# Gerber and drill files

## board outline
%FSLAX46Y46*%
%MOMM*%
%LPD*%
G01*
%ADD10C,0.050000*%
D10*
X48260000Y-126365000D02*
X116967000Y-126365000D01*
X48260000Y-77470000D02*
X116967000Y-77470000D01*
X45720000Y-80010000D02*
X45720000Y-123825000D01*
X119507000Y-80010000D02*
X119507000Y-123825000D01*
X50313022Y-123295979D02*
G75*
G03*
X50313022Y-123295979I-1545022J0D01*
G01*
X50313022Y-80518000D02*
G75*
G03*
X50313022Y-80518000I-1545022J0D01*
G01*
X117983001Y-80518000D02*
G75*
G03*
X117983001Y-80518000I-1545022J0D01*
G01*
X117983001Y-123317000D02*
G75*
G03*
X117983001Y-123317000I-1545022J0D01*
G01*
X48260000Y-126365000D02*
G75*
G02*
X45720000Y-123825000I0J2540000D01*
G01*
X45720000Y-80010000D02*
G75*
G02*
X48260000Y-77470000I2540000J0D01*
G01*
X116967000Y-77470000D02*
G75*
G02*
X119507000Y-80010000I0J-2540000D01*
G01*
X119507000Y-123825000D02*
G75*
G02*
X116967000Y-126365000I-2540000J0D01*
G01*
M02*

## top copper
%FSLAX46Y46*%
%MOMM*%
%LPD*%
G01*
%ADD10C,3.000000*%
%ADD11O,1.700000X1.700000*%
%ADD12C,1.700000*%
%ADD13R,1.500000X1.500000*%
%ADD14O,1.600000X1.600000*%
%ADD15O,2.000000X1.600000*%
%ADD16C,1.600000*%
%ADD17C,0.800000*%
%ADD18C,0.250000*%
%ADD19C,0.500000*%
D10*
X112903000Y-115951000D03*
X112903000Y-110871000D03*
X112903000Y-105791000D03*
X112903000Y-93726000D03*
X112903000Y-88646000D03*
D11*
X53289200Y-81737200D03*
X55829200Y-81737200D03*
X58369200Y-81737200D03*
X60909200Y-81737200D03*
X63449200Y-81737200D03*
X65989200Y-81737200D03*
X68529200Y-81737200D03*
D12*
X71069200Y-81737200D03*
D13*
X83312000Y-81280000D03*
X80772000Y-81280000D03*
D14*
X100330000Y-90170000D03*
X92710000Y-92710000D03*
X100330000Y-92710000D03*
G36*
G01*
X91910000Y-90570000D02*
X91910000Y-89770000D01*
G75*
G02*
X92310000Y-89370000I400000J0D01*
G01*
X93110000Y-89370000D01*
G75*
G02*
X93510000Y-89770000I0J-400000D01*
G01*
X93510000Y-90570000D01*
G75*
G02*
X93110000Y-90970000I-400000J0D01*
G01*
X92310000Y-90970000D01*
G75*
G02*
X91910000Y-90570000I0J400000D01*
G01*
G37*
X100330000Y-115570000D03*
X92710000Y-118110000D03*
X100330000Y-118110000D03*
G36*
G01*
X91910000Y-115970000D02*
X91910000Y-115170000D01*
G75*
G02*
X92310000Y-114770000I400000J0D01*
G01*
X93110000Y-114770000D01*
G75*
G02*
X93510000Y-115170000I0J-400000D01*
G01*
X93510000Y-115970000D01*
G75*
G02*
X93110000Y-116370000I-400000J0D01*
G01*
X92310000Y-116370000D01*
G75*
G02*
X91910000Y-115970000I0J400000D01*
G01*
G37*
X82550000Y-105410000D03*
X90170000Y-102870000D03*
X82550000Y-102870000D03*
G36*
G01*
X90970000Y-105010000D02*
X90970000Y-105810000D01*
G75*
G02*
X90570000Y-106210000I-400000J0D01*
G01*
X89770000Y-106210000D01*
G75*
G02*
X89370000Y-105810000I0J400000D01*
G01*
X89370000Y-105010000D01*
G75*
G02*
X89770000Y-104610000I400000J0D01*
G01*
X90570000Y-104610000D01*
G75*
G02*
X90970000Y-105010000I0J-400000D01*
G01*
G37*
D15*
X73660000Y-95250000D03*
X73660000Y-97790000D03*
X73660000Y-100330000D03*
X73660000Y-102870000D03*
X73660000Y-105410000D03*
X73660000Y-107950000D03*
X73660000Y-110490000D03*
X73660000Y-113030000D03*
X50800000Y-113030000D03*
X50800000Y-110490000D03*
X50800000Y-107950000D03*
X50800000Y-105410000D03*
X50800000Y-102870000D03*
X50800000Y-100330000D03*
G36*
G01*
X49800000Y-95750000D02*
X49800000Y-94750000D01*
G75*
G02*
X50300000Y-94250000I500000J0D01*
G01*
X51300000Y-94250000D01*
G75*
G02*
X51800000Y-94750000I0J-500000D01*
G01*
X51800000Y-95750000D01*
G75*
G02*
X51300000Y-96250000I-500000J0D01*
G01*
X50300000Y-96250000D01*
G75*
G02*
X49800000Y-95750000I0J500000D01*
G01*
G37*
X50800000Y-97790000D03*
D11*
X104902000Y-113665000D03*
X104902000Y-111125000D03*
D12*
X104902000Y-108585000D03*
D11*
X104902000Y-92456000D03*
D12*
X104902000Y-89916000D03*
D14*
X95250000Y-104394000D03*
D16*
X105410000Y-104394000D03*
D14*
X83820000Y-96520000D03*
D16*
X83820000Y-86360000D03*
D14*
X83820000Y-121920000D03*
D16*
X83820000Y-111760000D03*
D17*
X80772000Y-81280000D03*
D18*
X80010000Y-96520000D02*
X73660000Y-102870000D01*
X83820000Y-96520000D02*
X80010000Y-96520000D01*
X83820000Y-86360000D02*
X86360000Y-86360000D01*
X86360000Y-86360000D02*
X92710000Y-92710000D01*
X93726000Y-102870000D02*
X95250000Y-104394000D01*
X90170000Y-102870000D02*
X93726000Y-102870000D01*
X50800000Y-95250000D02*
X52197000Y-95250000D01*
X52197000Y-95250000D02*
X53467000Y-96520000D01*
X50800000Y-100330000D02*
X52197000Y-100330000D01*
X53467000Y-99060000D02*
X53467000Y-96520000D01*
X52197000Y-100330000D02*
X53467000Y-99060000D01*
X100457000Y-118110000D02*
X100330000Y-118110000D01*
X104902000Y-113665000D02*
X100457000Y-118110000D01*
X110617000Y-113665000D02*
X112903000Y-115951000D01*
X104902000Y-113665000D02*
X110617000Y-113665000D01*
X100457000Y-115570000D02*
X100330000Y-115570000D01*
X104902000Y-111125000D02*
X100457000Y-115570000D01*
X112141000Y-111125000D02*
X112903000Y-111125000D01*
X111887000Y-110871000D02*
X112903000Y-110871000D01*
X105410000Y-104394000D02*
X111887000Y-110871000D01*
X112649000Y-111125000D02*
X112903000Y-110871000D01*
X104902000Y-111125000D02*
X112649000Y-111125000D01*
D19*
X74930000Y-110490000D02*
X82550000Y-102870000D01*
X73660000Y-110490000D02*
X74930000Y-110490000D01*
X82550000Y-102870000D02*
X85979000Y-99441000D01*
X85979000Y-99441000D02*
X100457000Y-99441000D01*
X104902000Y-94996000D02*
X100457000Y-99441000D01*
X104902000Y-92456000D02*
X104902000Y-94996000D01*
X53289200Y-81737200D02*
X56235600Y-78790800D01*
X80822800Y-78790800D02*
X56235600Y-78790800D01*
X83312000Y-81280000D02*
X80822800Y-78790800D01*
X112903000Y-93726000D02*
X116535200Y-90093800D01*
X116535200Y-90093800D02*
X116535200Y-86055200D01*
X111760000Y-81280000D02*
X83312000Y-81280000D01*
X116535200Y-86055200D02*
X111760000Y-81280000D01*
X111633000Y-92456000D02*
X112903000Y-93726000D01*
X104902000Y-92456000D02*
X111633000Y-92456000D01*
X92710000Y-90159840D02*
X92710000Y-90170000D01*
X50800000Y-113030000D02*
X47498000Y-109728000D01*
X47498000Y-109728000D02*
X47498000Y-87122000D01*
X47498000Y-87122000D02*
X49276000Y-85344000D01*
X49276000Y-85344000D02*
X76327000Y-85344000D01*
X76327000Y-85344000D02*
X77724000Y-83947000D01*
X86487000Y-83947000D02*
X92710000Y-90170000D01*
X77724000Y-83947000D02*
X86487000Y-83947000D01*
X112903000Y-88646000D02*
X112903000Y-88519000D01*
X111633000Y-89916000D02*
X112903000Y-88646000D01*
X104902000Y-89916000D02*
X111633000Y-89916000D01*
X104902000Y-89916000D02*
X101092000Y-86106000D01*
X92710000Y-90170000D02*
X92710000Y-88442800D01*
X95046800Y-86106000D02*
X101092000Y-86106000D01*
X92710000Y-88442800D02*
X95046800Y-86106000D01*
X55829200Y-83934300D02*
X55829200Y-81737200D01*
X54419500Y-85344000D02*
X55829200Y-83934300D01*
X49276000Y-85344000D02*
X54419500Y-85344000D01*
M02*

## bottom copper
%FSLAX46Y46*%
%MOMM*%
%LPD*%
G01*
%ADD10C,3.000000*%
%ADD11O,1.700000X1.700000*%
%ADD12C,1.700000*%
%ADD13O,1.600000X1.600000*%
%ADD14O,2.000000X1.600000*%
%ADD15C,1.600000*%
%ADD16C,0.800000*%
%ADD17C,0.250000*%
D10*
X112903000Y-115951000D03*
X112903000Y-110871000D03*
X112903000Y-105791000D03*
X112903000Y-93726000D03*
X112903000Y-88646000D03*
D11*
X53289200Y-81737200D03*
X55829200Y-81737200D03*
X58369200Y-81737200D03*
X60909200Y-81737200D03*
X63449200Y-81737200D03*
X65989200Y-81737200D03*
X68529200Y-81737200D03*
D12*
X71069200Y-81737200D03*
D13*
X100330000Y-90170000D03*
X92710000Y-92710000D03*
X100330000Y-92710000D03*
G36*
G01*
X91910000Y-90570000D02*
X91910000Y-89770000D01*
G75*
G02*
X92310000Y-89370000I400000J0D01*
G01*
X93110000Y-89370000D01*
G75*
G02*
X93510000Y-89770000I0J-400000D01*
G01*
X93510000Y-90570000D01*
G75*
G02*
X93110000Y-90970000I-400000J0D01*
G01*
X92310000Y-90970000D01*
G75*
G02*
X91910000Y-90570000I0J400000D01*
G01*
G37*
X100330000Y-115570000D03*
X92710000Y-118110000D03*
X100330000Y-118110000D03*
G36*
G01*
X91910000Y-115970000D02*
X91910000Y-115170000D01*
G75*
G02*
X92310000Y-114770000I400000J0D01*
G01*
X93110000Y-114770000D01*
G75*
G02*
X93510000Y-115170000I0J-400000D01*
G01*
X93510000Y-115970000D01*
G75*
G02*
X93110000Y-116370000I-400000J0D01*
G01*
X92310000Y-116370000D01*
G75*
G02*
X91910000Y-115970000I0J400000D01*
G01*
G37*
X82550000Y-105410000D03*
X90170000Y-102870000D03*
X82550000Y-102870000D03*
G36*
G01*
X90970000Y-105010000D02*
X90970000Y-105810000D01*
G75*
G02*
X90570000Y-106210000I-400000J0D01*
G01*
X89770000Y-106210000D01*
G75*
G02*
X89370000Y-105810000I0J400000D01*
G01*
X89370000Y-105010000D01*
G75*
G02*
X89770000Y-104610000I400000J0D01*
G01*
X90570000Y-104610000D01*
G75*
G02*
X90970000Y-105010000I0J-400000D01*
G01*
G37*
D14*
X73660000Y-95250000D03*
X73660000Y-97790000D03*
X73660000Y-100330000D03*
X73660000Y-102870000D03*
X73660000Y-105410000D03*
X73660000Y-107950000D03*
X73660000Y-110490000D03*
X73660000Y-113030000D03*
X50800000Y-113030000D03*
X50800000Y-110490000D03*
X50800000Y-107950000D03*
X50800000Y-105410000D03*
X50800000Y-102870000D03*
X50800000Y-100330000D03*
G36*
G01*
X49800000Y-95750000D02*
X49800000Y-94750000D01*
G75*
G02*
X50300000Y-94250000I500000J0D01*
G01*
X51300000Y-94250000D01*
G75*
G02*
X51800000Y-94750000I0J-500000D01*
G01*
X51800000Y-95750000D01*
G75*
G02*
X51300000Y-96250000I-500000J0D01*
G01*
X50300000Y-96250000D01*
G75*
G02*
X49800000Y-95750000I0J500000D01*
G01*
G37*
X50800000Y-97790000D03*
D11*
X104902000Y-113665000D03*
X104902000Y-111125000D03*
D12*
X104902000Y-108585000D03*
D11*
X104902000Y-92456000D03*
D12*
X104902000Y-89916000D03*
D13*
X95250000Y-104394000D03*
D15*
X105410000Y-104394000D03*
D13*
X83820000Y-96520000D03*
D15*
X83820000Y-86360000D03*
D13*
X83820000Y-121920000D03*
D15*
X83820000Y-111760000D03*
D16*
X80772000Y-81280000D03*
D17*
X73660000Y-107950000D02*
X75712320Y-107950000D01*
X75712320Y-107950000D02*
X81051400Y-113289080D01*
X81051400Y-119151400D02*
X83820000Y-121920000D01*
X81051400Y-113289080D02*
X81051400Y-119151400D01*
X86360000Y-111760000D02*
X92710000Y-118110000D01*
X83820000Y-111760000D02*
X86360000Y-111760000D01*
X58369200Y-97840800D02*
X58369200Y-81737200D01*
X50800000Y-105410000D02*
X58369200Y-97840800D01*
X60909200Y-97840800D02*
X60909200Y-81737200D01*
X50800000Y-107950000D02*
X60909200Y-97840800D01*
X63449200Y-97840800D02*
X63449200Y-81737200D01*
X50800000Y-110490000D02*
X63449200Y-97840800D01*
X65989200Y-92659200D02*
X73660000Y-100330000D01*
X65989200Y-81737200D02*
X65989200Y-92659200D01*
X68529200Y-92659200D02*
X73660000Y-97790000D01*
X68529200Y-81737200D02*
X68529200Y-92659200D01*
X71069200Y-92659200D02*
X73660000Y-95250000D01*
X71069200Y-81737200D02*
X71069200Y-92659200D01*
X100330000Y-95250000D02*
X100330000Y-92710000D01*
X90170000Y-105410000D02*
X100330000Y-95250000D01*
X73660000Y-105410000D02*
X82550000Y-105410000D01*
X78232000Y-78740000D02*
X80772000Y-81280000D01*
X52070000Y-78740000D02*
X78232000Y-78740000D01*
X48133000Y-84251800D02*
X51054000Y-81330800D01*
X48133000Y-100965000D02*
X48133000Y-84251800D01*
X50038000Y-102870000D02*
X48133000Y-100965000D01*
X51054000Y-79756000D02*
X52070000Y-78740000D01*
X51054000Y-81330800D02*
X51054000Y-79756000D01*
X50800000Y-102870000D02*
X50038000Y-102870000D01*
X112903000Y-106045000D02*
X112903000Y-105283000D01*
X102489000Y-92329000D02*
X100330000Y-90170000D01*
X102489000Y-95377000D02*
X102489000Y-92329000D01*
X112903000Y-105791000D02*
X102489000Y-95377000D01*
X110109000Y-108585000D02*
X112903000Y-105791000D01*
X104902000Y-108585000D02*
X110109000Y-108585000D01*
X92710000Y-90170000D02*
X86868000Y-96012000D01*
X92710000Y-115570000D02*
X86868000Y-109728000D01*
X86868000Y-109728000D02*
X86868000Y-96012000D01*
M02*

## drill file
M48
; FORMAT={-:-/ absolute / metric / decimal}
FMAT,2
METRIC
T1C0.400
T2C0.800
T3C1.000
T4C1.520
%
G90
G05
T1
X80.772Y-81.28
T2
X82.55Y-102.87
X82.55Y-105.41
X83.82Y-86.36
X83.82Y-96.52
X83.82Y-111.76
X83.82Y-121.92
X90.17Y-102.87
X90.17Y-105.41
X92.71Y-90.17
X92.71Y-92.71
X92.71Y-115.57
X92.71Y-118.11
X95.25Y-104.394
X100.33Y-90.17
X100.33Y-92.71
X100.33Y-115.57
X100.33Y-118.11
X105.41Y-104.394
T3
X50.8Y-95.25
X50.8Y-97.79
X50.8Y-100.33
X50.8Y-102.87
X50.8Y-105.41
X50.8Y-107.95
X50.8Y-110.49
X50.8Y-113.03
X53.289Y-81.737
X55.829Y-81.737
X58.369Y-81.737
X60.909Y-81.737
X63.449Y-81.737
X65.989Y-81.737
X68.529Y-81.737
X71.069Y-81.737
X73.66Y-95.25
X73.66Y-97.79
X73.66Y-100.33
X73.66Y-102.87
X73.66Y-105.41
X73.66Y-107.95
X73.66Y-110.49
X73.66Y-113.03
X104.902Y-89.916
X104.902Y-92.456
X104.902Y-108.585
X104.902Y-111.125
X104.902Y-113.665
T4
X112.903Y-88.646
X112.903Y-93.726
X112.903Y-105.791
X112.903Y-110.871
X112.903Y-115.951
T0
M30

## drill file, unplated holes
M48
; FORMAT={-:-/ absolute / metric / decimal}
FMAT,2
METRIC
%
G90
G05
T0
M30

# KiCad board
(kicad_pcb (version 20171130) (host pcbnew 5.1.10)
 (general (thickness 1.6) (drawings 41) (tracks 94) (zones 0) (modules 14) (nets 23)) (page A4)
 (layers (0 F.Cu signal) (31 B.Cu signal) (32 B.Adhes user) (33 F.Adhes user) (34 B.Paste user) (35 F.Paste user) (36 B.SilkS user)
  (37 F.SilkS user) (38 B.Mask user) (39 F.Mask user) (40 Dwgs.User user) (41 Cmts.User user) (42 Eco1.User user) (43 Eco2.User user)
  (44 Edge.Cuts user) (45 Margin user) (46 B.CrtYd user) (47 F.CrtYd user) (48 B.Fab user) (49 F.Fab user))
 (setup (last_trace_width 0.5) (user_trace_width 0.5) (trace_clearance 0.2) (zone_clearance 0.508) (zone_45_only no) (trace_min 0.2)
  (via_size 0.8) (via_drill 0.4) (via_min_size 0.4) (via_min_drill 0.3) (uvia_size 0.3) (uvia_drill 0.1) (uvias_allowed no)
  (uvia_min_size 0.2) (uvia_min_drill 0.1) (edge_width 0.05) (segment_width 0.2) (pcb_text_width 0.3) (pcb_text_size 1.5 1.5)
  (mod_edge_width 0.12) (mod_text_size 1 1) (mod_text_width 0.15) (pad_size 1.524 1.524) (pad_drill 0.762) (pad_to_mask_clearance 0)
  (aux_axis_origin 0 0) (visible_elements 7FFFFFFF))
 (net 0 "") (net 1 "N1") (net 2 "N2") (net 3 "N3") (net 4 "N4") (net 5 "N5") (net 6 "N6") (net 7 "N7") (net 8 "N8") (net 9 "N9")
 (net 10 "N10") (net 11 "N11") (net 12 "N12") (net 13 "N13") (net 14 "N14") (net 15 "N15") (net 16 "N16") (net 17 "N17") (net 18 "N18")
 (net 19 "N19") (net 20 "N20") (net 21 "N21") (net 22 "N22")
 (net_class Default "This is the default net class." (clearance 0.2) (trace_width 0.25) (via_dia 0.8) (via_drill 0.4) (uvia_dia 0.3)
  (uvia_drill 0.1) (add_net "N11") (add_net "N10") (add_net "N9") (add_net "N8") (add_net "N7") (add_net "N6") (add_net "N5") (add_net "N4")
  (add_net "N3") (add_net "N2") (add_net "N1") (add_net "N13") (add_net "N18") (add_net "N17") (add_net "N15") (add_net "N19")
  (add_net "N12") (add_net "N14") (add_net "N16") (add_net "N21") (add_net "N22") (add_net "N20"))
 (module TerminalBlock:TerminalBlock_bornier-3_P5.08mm (layer F.Cu) (at 112.903 105.791 270)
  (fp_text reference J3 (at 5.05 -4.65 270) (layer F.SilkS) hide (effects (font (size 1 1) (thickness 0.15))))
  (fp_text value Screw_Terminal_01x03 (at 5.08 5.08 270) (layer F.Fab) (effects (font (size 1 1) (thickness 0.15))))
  (pad 3 thru_hole circle (at 10.16 0 270) (size 3 3) (drill 1.52) (layers *.Cu *.Mask) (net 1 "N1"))
  (pad 2 thru_hole circle (at 5.08 0 270) (size 3 3) (drill 1.52) (layers *.Cu *.Mask) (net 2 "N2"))
  (pad 1 thru_hole circle (at 0 0 270) (size 3 3) (drill 1.52) (layers *.Cu *.Mask) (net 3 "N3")))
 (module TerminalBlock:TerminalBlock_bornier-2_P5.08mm (layer F.Cu) (at 112.903 88.646 270)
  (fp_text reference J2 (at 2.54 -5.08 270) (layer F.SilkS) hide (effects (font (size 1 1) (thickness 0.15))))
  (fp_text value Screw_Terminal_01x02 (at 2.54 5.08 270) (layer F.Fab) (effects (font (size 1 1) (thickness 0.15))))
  (pad 2 thru_hole circle (at 5.08 0 270) (size 3 3) (drill 1.52) (layers *.Cu *.Mask) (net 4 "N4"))
  (pad 1 thru_hole circle (at 0 0 270) (size 3 3) (drill 1.52) (layers *.Cu *.Mask) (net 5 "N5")))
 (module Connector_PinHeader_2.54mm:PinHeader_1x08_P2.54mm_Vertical (layer F.Cu) (at 71.0692 81.7372 270)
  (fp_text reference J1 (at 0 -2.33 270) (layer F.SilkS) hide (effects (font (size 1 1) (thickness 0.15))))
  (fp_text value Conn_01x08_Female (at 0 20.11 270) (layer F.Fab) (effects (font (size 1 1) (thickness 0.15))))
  (pad 8 thru_hole oval (at 0 17.78 270) (size 1.7 1.7) (drill 1) (layers *.Cu *.Mask) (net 4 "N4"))
  (pad 7 thru_hole oval (at 0 15.24 270) (size 1.7 1.7) (drill 1) (layers *.Cu *.Mask) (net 5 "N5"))
  (pad 6 thru_hole oval (at 0 12.7 270) (size 1.7 1.7) (drill 1) (layers *.Cu *.Mask) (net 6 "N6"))
  (pad 5 thru_hole oval (at 0 10.16 270) (size 1.7 1.7) (drill 1) (layers *.Cu *.Mask) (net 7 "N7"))
  (pad 4 thru_hole oval (at 0 7.62 270) (size 1.7 1.7) (drill 1) (layers *.Cu *.Mask) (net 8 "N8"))
  (pad 3 thru_hole oval (at 0 5.08 270) (size 1.7 1.7) (drill 1) (layers *.Cu *.Mask) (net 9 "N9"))
  (pad 2 thru_hole oval (at 0 2.54 270) (size 1.7 1.7) (drill 1) (layers *.Cu *.Mask) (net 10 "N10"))
  (pad 1 thru_hole circle (at 0 0 270) (size 1.7 1.7) (drill 1) (layers *.Cu *.Mask) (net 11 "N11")))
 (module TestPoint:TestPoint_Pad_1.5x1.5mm (layer F.Cu) (at 83.312 81.28)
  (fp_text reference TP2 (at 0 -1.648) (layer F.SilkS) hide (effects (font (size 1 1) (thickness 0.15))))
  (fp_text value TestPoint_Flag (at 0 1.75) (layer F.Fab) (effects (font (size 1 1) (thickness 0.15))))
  (pad 1 smd rect (at 0 0) (size 1.5 1.5) (layers F.Cu F.Mask) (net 4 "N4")))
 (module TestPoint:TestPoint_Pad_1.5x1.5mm (layer F.Cu) (at 80.772 81.28)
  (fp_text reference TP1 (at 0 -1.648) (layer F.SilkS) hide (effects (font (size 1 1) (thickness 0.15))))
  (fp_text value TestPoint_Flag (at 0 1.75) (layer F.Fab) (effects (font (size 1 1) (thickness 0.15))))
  (pad 1 smd rect (at 0 0) (size 1.5 1.5) (layers F.Cu F.Mask) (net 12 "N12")))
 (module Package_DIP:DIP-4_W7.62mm (layer F.Cu) (at 92.71 90.17)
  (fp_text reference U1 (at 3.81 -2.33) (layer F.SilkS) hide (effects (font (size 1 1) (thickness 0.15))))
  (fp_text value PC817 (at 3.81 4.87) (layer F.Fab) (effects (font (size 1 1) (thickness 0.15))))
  (pad 4 thru_hole oval (at 7.62 0) (size 1.6 1.6) (drill 0.8) (layers *.Cu *.Mask) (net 3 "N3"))
  (pad 2 thru_hole oval (at 0 2.54) (size 1.6 1.6) (drill 0.8) (layers *.Cu *.Mask) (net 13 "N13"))
  (pad 3 thru_hole oval (at 7.62 2.54) (size 1.6 1.6) (drill 0.8) (layers *.Cu *.Mask) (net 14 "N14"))
  (pad 1 thru_hole roundrect (at 0 0) (size 1.6 1.6) (drill 0.8) (layers *.Cu *.Mask) (roundrect_rratio 0.25) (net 5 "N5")))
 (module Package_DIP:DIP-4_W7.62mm (layer F.Cu) (at 92.71 115.57)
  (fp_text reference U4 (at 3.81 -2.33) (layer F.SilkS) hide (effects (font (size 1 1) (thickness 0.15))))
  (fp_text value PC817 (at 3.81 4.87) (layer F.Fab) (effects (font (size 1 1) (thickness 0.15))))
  (pad 4 thru_hole oval (at 7.62 0) (size 1.6 1.6) (drill 0.8) (layers *.Cu *.Mask) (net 2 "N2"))
  (pad 2 thru_hole oval (at 0 2.54) (size 1.6 1.6) (drill 0.8) (layers *.Cu *.Mask) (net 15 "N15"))
  (pad 3 thru_hole oval (at 7.62 2.54) (size 1.6 1.6) (drill 0.8) (layers *.Cu *.Mask) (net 1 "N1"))
  (pad 1 thru_hole roundrect (at 0 0) (size 1.6 1.6) (drill 0.8) (layers *.Cu *.Mask) (roundrect_rratio 0.25) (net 5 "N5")))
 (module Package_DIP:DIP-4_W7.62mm (layer F.Cu) (at 90.17 105.41 180)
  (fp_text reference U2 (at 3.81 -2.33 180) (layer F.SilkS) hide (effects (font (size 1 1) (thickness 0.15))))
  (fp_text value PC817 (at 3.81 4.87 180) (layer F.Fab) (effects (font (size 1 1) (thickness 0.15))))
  (pad 4 thru_hole oval (at 7.62 0 180) (size 1.6 1.6) (drill 0.8) (layers *.Cu *.Mask) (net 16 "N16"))
  (pad 2 thru_hole oval (at 0 2.54 180) (size 1.6 1.6) (drill 0.8) (layers *.Cu *.Mask) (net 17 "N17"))
  (pad 3 thru_hole oval (at 7.62 2.54 180) (size 1.6 1.6) (drill 0.8) (layers *.Cu *.Mask) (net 4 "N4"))
  (pad 1 thru_hole roundrect (at 0 0 180) (size 1.6 1.6) (drill 0.8) (layers *.Cu *.Mask) (roundrect_rratio 0.25) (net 14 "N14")))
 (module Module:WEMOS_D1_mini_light (layer F.Cu) (at 50.8 95.25)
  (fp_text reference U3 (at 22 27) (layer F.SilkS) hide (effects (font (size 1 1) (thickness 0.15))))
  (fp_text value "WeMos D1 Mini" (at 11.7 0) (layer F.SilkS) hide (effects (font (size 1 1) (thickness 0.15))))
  (pad 16 thru_hole oval (at 22.86 0) (size 2 1.6) (drill 1) (layers *.Cu *.Mask) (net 11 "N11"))
  (pad 15 thru_hole oval (at 22.86 2.54) (size 2 1.6) (drill 1) (layers *.Cu *.Mask) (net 10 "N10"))
  (pad 14 thru_hole oval (at 22.86 5.08) (size 2 1.6) (drill 1) (layers *.Cu *.Mask) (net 9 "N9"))
  (pad 13 thru_hole oval (at 22.86 7.62) (size 2 1.6) (drill 1) (layers *.Cu *.Mask) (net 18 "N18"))
  (pad 12 thru_hole oval (at 22.86 10.16) (size 2 1.6) (drill 1) (layers *.Cu *.Mask) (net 16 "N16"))
  (pad 11 thru_hole oval (at 22.86 12.7) (size 2 1.6) (drill 1) (layers *.Cu *.Mask) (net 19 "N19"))
  (pad 10 thru_hole oval (at 22.86 15.24) (size 2 1.6) (drill 1) (layers *.Cu *.Mask) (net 4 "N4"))
  (pad 9 thru_hole oval (at 22.86 17.78) (size 2 1.6) (drill 1) (layers *.Cu *.Mask) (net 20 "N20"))
  (pad 8 thru_hole oval (at 0 17.78) (size 2 1.6) (drill 1) (layers *.Cu *.Mask) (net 5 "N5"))
  (pad 7 thru_hole oval (at 0 15.24) (size 2 1.6) (drill 1) (layers *.Cu *.Mask) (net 8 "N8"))
  (pad 6 thru_hole oval (at 0 12.7) (size 2 1.6) (drill 1) (layers *.Cu *.Mask) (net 7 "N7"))
  (pad 5 thru_hole oval (at 0 10.16) (size 2 1.6) (drill 1) (layers *.Cu *.Mask) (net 6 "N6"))
  (pad 4 thru_hole oval (at 0 7.62) (size 2 1.6) (drill 1) (layers *.Cu *.Mask) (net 12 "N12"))
  (pad 3 thru_hole oval (at 0 5.08) (size 2 1.6) (drill 1) (layers *.Cu *.Mask) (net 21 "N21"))
  (pad 1 thru_hole roundrect (at 0 0) (size 2 2) (drill 1) (layers *.Cu *.Mask) (roundrect_rratio 0.25) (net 21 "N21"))
  (pad 2 thru_hole oval (at 0 2.54) (size 2 1.6) (drill 1) (layers *.Cu *.Mask) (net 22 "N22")))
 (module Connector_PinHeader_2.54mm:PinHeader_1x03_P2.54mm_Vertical (layer F.Cu) (at 104.902 108.585)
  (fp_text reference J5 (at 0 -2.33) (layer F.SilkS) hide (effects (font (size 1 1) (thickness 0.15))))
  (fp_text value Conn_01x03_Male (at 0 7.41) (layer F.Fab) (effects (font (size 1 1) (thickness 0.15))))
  (pad 3 thru_hole oval (at 0 5.08) (size 1.7 1.7) (drill 1) (layers *.Cu *.Mask) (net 1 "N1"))
  (pad 2 thru_hole oval (at 0 2.54) (size 1.7 1.7) (drill 1) (layers *.Cu *.Mask) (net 2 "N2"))
  (pad 1 thru_hole circle (at 0 0) (size 1.7 1.7) (drill 1) (layers *.Cu *.Mask) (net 3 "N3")))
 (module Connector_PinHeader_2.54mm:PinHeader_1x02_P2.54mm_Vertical (layer F.Cu) (at 104.902 89.916)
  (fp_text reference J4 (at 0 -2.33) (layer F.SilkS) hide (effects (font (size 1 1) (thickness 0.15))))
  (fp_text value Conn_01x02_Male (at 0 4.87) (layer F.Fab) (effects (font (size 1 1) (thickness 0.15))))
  (pad 2 thru_hole oval (at 0 2.54) (size 1.7 1.7) (drill 1) (layers *.Cu *.Mask) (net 4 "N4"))
  (pad 1 thru_hole circle (at 0 0) (size 1.7 1.7) (drill 1) (layers *.Cu *.Mask) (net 5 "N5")))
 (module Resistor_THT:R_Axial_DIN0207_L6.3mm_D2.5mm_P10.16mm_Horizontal (layer F.Cu) (at 105.41 104.394 180)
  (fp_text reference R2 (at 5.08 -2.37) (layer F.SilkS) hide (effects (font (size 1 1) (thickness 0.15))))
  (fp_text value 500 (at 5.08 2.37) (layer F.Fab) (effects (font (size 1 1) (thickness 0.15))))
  (pad 2 thru_hole oval (at 10.16 0 180) (size 1.6 1.6) (drill 0.8) (layers *.Cu *.Mask) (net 17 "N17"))
  (pad 1 thru_hole circle (at 0 0 180) (size 1.6 1.6) (drill 0.8) (layers *.Cu *.Mask) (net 2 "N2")))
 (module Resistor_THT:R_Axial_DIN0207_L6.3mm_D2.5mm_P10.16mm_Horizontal (layer F.Cu) (at 83.82 86.36 270)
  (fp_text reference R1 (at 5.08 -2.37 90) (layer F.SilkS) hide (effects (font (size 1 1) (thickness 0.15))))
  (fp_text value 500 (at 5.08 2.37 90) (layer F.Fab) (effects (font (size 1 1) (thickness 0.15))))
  (pad 2 thru_hole oval (at 10.16 0 270) (size 1.6 1.6) (drill 0.8) (layers *.Cu *.Mask) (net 18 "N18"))
  (pad 1 thru_hole circle (at 0 0 270) (size 1.6 1.6) (drill 0.8) (layers *.Cu *.Mask) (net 13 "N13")))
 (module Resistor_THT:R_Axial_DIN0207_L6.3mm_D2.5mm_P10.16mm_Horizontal (layer F.Cu) (at 83.82 111.76 270)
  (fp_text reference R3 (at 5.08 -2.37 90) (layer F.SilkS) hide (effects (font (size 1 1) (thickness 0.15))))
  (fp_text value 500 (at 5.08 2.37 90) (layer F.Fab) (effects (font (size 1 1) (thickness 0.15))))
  (pad 2 thru_hole oval (at 10.16 0 270) (size 1.6 1.6) (drill 0.8) (layers *.Cu *.Mask) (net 19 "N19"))
  (pad 1 thru_hole circle (at 0 0 270) (size 1.6 1.6) (drill 0.8) (layers *.Cu *.Mask) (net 15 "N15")))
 (gr_line (start 48.26 126.365) (end 116.967 126.365) (layer Edge.Cuts) (width 0.05))
 (gr_line (start 48.26 77.47) (end 116.967 77.47) (layer Edge.Cuts) (width 0.05))
 (gr_line (start 45.72 80.01) (end 45.72 123.825) (layer Edge.Cuts) (width 0.05))
 (gr_line (start 119.507 80.01) (end 119.507 123.825) (layer Edge.Cuts) (width 0.05))
 (gr_circle (center 48.768 123.295979) (end 50.292 123.041979) (layer Edge.Cuts) (width 0.05))
 (gr_circle (center 48.768 80.518) (end 50.292 80.264) (layer Edge.Cuts) (width 0.05))
 (gr_circle (center 116.437979 80.518) (end 117.961979 80.264) (layer Edge.Cuts) (width 0.05))
 (gr_circle (center 116.437979 123.317) (end 117.961979 123.063) (layer Edge.Cuts) (width 0.05))
 (gr_arc (start 48.26 123.825) (end 45.72 123.825) (angle -90) (layer Edge.Cuts) (width 0.05))
 (gr_arc (start 48.26 80.01) (end 48.26 77.47) (angle -90) (layer Edge.Cuts) (width 0.05))
 (gr_arc (start 116.967 80.01) (end 119.507 80.01) (angle -90) (layer Edge.Cuts) (width 0.05))
 (gr_arc (start 116.967 123.825) (end 116.967 126.365) (angle -90) (layer Edge.Cuts) (width 0.05))
 (segment (start 80.01 96.52) (end 73.66 102.87) (width 0.25) (layer F.Cu) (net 18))
 (segment (start 83.82 96.52) (end 80.01 96.52) (width 0.25) (layer F.Cu) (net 18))
 (segment (start 83.82 86.36) (end 86.36 86.36) (width 0.25) (layer F.Cu) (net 13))
 (segment (start 86.36 86.36) (end 92.71 92.71) (width 0.25) (layer F.Cu) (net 13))
 (segment (start 93.726 102.87) (end 95.25 104.394) (width 0.25) (layer F.Cu) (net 17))
 (segment (start 90.17 102.87) (end 93.726 102.87) (width 0.25) (layer F.Cu) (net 17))
 (segment (start 73.66 107.95) (end 75.71232 107.95) (width 0.25) (layer B.Cu) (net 19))
 (segment (start 75.71232 107.95) (end 81.0514 113.28908) (width 0.25) (layer B.Cu) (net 19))
 (segment (start 81.0514 119.1514) (end 83.82 121.92) (width 0.25) (layer B.Cu) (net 19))
 (segment (start 81.0514 113.28908) (end 81.0514 119.1514) (width 0.25) (layer B.Cu) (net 19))
 (segment (start 86.36 111.76) (end 92.71 118.11) (width 0.25) (layer B.Cu) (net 15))
 (segment (start 83.82 111.76) (end 86.36 111.76) (width 0.25) (layer B.Cu) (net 15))
 (segment (start 58.3692 97.8408) (end 58.3692 81.7372) (width 0.25) (layer B.Cu) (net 6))
 (segment (start 50.8 105.41) (end 58.3692 97.8408) (width 0.25) (layer B.Cu) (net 6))
 (segment (start 60.9092 97.8408) (end 60.9092 81.7372) (width 0.25) (layer B.Cu) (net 7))
 (segment (start 50.8 107.95) (end 60.9092 97.8408) (width 0.25) (layer B.Cu) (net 7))
 (segment (start 63.4492 97.8408) (end 63.4492 81.7372) (width 0.25) (layer B.Cu) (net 8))
 (segment (start 50.8 110.49) (end 63.4492 97.8408) (width 0.25) (layer B.Cu) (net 8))
 (segment (start 65.9892 92.6592) (end 73.66 100.33) (width 0.25) (layer B.Cu) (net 9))
 (segment (start 65.9892 81.7372) (end 65.9892 92.6592) (width 0.25) (layer B.Cu) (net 9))
 (segment (start 68.5292 92.6592) (end 73.66 97.79) (width 0.25) (layer B.Cu) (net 10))
 (segment (start 68.5292 81.7372) (end 68.5292 92.6592) (width 0.25) (layer B.Cu) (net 10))
 (segment (start 71.0692 92.6592) (end 73.66 95.25) (width 0.25) (layer B.Cu) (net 11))
 (segment (start 71.0692 81.7372) (end 71.0692 92.6592) (width 0.25) (layer B.Cu) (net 11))
 (segment (start 100.33 95.25) (end 100.33 92.71) (width 0.25) (layer B.Cu) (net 14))
 (segment (start 90.17 105.41) (end 100.33 95.25) (width 0.25) (layer B.Cu) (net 14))
 (segment (start 73.66 105.41) (end 82.55 105.41) (width 0.25) (layer B.Cu) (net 16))
 (segment (start 50.8 95.25) (end 52.197 95.25) (width 0.25) (layer F.Cu) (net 21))
 (segment (start 52.197 95.25) (end 53.467 96.52) (width 0.25) (layer F.Cu) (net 21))
 (segment (start 50.8 100.33) (end 52.197 100.33) (width 0.25) (layer F.Cu) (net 21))
 (segment (start 53.467 99.06) (end 53.467 96.52) (width 0.25) (layer F.Cu) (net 21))
 (segment (start 52.197 100.33) (end 53.467 99.06) (width 0.25) (layer F.Cu) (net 21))
 (via (at 80.772 81.28) (size 0.8) (drill 0.4) (layers F.Cu B.Cu) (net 12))
 (segment (start 78.232 78.74) (end 80.772 81.28) (width 0.25) (layer B.Cu) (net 12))
 (segment (start 52.07 78.74) (end 78.232 78.74) (width 0.25) (layer B.Cu) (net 12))
 (segment (start 48.133 84.2518) (end 51.054 81.3308) (width 0.25) (layer B.Cu) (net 12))
 (segment (start 48.133 100.965) (end 48.133 84.2518) (width 0.25) (layer B.Cu) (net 12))
 (segment (start 50.038 102.87) (end 48.133 100.965) (width 0.25) (layer B.Cu) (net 12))
 (segment (start 51.054 79.756) (end 52.07 78.74) (width 0.25) (layer B.Cu) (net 12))
 (segment (start 51.054 81.3308) (end 51.054 79.756) (width 0.25) (layer B.Cu) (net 12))
 (segment (start 50.8 102.87) (end 50.038 102.87) (width 0.25) (layer B.Cu) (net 12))
 (segment (start 100.457 118.11) (end 100.33 118.11) (width 0.25) (layer F.Cu) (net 1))
 (segment (start 104.902 113.665) (end 100.457 118.11) (width 0.25) (layer F.Cu) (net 1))
 (segment (start 110.617 113.665) (end 112.903 115.951) (width 0.25) (layer F.Cu) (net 1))
 (segment (start 104.902 113.665) (end 110.617 113.665) (width 0.25) (layer F.Cu) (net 1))
 (segment (start 100.457 115.57) (end 100.33 115.57) (width 0.25) (layer F.Cu) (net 2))
 (segment (start 104.902 111.125) (end 100.457 115.57) (width 0.25) (layer F.Cu) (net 2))
 (segment (start 112.141 111.125) (end 112.903 111.125) (width 0.25) (layer F.Cu) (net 2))
 (segment (start 111.887 110.871) (end 112.903 110.871) (width 0.25) (layer F.Cu) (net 2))
 (segment (start 105.41 104.394) (end 111.887 110.871) (width 0.25) (layer F.Cu) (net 2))
 (segment (start 112.649 111.125) (end 112.903 110.871) (width 0.25) (layer F.Cu) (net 2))
 (segment (start 104.902 111.125) (end 112.649 111.125) (width 0.25) (layer F.Cu) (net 2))
 (segment (start 112.903 106.045) (end 112.903 105.283) (width 0.25) (layer B.Cu) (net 3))
 (segment (start 102.489 92.329) (end 100.33 90.17) (width 0.25) (layer B.Cu) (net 3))
 (segment (start 102.489 95.377) (end 102.489 92.329) (width 0.25) (layer B.Cu) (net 3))
 (segment (start 112.903 105.791) (end 102.489 95.377) (width 0.25) (layer B.Cu) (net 3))
 (segment (start 110.109 108.585) (end 112.903 105.791) (width 0.25) (layer B.Cu) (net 3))
 (segment (start 104.902 108.585) (end 110.109 108.585) (width 0.25) (layer B.Cu) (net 3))
 (segment (start 74.93 110.49) (end 82.55 102.87) (width 0.5) (layer F.Cu) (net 4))
 (segment (start 73.66 110.49) (end 74.93 110.49) (width 0.5) (layer F.Cu) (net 4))
 (segment (start 82.55 102.87) (end 85.979 99.441) (width 0.5) (layer F.Cu) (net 4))
 (segment (start 85.979 99.441) (end 100.457 99.441) (width 0.5) (layer F.Cu) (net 4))
 (segment (start 104.902 94.996) (end 100.457 99.441) (width 0.5) (layer F.Cu) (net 4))
 (segment (start 104.902 92.456) (end 104.902 94.996) (width 0.5) (layer F.Cu) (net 4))
 (segment (start 53.2892 81.7372) (end 56.2356 78.7908) (width 0.5) (layer F.Cu) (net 4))
 (segment (start 80.8228 78.7908) (end 56.2356 78.7908) (width 0.5) (layer F.Cu) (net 4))
 (segment (start 83.312 81.28) (end 80.8228 78.7908) (width 0.5) (layer F.Cu) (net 4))
 (segment (start 112.903 93.726) (end 116.5352 90.0938) (width 0.5) (layer F.Cu) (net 4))
 (segment (start 116.5352 90.0938) (end 116.5352 86.0552) (width 0.5) (layer F.Cu) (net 4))
 (segment (start 111.76 81.28) (end 83.312 81.28) (width 0.5) (layer F.Cu) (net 4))
 (segment (start 116.5352 86.0552) (end 111.76 81.28) (width 0.5) (layer F.Cu) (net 4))
 (segment (start 111.633 92.456) (end 112.903 93.726) (width 0.5) (layer F.Cu) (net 4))
 (segment (start 104.902 92.456) (end 111.633 92.456) (width 0.5) (layer F.Cu) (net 4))
 (segment (start 92.71 90.17) (end 86.868 96.012) (width 0.25) (layer B.Cu) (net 5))
 (segment (start 92.71 115.57) (end 86.868 109.728) (width 0.25) (layer B.Cu) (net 5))
 (segment (start 86.868 109.728) (end 86.868 96.012) (width 0.25) (layer B.Cu) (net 5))
 (segment (start 92.71 90.15984) (end 92.71 90.17) (width 0.5) (layer F.Cu) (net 5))
 (segment (start 50.8 113.03) (end 47.498 109.728) (width 0.5) (layer F.Cu) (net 5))
 (segment (start 47.498 109.728) (end 47.498 87.122) (width 0.5) (layer F.Cu) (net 5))
 (segment (start 47.498 87.122) (end 49.276 85.344) (width 0.5) (layer F.Cu) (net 5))
 (segment (start 49.276 85.344) (end 76.327 85.344) (width 0.5) (layer F.Cu) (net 5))
 (segment (start 76.327 85.344) (end 77.724 83.947) (width 0.5) (layer F.Cu) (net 5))
 (segment (start 86.487 83.947) (end 92.71 90.17) (width 0.5) (layer F.Cu) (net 5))
 (segment (start 77.724 83.947) (end 86.487 83.947) (width 0.5) (layer F.Cu) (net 5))
 (segment (start 112.903 88.646) (end 112.903 88.519) (width 0.5) (layer F.Cu) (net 5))
 (segment (start 111.633 89.916) (end 112.903 88.646) (width 0.5) (layer F.Cu) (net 5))
 (segment (start 104.902 89.916) (end 111.633 89.916) (width 0.5) (layer F.Cu) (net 5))
 (segment (start 104.902 89.916) (end 101.092 86.106) (width 0.5) (layer F.Cu) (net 5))
 (segment (start 92.71 90.17) (end 92.71 88.4428) (width 0.5) (layer F.Cu) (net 5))
 (segment (start 95.0468 86.106) (end 101.092 86.106) (width 0.5) (layer F.Cu) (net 5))
 (segment (start 92.71 88.4428) (end 95.0468 86.106) (width 0.5) (layer F.Cu) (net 5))
 (segment (start 55.8292 83.9343) (end 55.8292 81.7372) (width 0.5) (layer F.Cu) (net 5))
 (segment (start 54.4195 85.344) (end 55.8292 83.9343) (width 0.5) (layer F.Cu) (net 5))
 (segment (start 49.276 85.344) (end 54.4195 85.344) (width 0.5) (layer F.Cu) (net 5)))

